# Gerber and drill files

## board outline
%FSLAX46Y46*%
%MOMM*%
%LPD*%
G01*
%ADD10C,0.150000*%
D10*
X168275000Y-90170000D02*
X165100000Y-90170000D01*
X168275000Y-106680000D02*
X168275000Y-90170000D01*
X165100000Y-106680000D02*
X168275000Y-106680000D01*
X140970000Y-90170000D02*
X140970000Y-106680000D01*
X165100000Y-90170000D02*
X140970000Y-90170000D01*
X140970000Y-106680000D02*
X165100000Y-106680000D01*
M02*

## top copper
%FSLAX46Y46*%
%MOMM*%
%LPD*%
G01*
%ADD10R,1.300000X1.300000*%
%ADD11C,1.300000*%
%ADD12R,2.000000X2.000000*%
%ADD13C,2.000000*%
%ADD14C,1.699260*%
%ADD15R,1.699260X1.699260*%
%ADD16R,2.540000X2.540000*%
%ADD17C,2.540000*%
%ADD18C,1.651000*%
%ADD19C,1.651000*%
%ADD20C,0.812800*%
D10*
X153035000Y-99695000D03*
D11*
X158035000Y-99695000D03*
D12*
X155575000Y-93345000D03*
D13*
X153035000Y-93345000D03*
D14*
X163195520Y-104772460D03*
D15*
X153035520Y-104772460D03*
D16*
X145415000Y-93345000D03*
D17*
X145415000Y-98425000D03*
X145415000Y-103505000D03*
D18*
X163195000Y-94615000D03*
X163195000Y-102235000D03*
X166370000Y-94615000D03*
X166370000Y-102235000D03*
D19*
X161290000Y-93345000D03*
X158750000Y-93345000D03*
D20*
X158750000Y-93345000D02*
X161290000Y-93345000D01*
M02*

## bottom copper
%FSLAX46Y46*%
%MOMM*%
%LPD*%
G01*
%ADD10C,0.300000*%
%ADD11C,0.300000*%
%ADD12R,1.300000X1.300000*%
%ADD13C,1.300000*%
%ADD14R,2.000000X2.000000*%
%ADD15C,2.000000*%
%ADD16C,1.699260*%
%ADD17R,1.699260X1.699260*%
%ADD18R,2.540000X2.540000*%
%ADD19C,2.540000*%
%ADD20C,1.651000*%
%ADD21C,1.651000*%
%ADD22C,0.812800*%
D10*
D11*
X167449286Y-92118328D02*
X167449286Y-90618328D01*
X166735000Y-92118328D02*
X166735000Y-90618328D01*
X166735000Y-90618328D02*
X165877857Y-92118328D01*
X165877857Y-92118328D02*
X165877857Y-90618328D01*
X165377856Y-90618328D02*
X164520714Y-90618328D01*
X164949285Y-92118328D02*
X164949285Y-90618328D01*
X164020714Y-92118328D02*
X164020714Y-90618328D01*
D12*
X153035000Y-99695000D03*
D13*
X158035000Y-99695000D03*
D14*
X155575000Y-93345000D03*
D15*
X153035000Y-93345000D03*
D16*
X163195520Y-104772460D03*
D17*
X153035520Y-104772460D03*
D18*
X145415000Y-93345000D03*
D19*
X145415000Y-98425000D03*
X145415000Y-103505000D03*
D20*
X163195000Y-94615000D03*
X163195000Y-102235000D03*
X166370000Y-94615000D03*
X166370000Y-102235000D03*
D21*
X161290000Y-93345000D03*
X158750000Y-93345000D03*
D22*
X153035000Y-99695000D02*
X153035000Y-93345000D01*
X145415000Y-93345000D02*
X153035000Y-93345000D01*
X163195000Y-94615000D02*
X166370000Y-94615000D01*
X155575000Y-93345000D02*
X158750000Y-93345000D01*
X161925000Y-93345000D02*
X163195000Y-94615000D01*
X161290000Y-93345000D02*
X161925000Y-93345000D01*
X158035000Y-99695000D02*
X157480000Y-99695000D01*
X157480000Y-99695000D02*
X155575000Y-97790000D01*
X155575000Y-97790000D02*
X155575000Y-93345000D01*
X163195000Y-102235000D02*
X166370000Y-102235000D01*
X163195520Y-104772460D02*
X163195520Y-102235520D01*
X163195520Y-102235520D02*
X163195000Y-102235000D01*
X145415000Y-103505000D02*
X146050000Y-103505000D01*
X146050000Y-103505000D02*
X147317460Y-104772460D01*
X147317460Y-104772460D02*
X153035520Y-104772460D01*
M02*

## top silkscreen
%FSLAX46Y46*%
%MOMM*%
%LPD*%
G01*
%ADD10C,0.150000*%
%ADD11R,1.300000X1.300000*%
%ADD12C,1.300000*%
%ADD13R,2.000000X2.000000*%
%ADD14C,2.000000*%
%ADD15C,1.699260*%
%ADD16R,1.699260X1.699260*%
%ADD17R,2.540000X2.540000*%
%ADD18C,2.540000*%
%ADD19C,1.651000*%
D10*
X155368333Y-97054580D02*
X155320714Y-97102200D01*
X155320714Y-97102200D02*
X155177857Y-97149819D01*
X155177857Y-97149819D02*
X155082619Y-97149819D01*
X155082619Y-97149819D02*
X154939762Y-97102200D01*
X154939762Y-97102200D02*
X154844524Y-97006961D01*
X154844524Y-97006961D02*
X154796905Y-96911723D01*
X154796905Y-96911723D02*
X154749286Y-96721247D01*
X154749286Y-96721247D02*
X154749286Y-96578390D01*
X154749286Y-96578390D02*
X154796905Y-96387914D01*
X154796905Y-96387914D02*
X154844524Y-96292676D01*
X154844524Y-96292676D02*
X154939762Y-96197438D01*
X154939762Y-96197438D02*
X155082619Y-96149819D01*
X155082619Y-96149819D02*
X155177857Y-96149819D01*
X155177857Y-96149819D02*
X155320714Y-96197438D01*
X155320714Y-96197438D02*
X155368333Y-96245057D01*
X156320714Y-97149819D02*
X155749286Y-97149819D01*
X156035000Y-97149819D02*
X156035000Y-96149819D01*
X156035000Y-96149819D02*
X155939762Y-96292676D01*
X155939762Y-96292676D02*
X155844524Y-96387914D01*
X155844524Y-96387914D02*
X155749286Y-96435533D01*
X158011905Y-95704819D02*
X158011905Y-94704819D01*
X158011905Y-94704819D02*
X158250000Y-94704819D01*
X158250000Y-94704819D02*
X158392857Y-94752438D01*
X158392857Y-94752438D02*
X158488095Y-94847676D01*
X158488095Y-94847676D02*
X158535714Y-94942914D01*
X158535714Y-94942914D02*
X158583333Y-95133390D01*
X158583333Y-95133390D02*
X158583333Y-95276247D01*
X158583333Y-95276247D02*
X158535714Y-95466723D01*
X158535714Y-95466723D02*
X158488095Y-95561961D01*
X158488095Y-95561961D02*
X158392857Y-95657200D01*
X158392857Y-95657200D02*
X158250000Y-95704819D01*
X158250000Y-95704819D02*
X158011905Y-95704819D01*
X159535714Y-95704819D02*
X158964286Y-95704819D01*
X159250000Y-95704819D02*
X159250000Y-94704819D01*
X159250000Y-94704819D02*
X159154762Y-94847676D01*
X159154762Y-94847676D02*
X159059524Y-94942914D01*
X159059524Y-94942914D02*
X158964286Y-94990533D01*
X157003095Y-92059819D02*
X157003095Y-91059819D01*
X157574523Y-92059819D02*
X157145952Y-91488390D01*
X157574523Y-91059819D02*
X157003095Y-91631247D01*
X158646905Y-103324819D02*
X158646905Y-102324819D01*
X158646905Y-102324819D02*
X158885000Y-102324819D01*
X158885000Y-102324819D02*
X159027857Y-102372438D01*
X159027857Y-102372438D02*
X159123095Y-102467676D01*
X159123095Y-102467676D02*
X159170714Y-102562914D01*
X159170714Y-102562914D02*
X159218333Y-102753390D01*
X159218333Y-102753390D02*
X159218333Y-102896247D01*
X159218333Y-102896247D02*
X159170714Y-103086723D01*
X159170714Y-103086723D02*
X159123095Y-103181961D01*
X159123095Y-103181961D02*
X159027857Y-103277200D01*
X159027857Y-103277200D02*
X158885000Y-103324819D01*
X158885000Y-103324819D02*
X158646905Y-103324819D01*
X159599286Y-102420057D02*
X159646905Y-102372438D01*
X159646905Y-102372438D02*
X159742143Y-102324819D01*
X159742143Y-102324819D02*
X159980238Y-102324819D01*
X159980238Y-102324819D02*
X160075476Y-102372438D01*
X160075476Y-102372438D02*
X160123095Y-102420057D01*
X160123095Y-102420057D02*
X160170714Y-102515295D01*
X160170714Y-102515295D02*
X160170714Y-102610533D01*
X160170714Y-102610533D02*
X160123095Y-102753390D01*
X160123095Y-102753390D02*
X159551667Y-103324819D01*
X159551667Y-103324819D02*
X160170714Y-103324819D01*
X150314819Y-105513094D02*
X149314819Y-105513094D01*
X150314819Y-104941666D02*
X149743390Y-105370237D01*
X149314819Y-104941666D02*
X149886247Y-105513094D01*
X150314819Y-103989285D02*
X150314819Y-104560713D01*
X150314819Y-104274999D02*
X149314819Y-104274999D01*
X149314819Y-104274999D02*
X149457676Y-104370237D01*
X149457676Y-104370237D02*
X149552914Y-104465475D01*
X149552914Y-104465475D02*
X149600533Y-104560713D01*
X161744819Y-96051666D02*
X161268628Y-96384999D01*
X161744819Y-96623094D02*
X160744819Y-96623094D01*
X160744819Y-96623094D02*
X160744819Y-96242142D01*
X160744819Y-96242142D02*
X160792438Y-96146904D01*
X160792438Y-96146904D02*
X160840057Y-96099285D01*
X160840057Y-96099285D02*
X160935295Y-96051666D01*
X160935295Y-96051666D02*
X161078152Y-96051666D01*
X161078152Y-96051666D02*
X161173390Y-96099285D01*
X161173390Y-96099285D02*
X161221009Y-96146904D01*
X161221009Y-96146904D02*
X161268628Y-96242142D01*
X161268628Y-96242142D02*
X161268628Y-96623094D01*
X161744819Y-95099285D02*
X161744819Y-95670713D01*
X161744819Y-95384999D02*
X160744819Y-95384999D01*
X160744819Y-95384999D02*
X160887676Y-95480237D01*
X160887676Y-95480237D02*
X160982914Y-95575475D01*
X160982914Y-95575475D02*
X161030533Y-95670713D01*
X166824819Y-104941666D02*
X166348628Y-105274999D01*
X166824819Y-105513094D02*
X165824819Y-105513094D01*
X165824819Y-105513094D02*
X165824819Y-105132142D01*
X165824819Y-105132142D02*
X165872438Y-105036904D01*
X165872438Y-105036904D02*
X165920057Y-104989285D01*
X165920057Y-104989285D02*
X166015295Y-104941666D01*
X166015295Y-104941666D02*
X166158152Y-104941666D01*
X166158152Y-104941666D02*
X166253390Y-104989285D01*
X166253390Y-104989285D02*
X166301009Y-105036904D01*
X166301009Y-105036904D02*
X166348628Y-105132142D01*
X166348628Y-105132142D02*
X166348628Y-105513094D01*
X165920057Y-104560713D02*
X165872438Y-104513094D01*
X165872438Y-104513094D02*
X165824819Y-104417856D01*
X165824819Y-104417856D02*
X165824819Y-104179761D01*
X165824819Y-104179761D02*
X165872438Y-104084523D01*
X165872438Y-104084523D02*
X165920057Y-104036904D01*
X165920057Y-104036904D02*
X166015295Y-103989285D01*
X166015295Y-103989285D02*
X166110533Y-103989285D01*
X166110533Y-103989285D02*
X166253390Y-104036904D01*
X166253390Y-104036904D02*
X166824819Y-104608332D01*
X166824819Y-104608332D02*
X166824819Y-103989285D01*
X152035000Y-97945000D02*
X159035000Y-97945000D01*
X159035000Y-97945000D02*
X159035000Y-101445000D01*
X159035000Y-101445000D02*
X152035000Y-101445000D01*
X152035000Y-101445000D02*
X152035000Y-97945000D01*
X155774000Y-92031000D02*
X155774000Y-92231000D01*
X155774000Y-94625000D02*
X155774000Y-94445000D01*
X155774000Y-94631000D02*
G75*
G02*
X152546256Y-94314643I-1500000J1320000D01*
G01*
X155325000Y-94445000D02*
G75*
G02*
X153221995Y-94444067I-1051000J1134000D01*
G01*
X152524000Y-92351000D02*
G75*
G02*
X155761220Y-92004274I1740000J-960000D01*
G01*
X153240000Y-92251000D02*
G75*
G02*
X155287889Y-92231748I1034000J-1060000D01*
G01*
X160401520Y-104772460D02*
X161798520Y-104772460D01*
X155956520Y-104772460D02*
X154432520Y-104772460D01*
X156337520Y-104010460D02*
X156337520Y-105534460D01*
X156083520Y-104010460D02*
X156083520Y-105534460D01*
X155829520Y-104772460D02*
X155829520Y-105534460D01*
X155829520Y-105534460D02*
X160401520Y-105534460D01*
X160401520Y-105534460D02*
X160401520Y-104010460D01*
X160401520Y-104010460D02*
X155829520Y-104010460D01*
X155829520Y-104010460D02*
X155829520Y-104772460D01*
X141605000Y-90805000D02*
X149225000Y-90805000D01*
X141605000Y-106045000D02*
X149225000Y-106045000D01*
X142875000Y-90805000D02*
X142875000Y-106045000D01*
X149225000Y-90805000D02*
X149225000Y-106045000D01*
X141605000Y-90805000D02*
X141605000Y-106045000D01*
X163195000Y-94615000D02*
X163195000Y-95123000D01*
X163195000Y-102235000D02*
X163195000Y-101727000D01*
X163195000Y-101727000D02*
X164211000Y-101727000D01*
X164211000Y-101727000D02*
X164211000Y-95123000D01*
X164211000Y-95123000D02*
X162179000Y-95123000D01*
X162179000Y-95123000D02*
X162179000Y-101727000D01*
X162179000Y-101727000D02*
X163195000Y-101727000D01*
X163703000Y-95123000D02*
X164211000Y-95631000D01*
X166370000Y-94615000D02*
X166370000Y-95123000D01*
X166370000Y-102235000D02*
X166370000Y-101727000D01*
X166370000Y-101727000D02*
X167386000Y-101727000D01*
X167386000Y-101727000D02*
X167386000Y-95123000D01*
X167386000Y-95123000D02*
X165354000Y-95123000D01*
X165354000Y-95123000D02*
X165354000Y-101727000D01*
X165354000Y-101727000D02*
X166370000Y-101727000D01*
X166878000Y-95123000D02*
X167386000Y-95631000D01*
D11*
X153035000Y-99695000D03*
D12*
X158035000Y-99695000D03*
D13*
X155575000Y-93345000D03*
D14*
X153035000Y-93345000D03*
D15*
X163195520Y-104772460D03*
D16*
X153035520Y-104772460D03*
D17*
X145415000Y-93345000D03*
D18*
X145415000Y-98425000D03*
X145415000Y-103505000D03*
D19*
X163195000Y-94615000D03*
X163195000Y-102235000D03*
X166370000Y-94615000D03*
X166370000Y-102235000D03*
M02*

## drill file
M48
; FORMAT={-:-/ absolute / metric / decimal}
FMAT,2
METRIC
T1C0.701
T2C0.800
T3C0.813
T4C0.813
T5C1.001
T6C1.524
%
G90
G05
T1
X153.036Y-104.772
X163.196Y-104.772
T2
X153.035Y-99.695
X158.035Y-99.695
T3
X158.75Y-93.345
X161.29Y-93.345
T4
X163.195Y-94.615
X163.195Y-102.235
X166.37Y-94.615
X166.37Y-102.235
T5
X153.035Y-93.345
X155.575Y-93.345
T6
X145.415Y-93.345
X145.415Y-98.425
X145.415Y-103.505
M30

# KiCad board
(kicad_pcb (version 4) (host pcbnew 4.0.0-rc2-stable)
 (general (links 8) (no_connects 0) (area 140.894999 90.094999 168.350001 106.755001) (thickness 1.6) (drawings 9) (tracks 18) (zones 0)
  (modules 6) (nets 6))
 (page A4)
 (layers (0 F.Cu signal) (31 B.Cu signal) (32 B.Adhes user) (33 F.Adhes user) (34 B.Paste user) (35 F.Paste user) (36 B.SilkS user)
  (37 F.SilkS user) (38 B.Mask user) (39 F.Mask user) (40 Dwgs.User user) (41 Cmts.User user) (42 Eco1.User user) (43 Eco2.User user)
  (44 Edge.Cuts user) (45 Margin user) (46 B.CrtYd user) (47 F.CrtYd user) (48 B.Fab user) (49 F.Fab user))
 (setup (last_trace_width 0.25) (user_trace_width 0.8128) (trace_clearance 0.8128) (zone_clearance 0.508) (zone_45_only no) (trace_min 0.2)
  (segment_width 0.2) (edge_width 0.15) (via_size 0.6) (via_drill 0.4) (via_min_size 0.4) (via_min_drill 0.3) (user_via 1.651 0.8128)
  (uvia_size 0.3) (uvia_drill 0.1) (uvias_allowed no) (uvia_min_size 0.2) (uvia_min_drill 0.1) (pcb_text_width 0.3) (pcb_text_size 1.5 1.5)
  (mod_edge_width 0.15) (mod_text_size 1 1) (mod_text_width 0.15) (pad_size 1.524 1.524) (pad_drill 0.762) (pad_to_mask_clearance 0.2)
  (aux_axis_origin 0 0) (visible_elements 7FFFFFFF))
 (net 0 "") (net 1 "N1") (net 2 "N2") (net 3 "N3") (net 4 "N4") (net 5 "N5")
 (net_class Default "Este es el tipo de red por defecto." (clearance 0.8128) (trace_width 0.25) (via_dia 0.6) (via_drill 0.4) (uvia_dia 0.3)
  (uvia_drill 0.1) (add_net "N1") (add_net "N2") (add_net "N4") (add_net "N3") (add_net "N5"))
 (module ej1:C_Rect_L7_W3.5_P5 (layer F.Cu) (at 153.035 99.695)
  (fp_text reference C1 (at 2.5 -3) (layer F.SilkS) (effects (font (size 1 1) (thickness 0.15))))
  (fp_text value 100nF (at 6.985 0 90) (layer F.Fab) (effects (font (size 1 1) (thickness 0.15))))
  (fp_line (start -1 -1.75) (end 6 -1.75) (layer F.SilkS) (width 0.15))
  (fp_line (start 6 -1.75) (end 6 1.75) (layer F.SilkS) (width 0.15))
  (fp_line (start 6 1.75) (end -1 1.75) (layer F.SilkS) (width 0.15))
  (fp_line (start -1 1.75) (end -1 -1.75) (layer F.SilkS) (width 0.15))
  (pad 1 thru_hole rect (at 0 0) (size 1.3 1.3) (drill 0.8) (layers *.Cu *.Mask F.SilkS) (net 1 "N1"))
  (pad 2 thru_hole circle (at 5 0) (size 1.3 1.3) (drill 0.8) (layers *.Cu *.Mask F.SilkS) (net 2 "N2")))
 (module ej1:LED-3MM (layer F.Cu) (at 155.575 93.345 180)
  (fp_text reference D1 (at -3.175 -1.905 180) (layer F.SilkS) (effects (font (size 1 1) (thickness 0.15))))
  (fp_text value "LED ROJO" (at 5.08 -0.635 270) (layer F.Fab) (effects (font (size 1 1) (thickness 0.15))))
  (fp_line (start -0.199 1.314) (end -0.199 1.114) (layer F.SilkS) (width 0.15))
  (fp_line (start -0.199 -1.28) (end -0.199 -1.1) (layer F.SilkS) (width 0.15))
  (fp_arc (start 1.301 0.034) (end -0.199 -1.286) (angle 108.5) (layer F.SilkS) (width 0.15))
  (fp_arc (start 1.301 0.034) (end 0.25 -1.1) (angle 85.7) (layer F.SilkS) (width 0.15))
  (fp_arc (start 1.311 0.034) (end 3.051 0.994) (angle 110) (layer F.SilkS) (width 0.15))
  (fp_arc (start 1.301 0.034) (end 2.335 1.094) (angle 87.5) (layer F.SilkS) (width 0.15))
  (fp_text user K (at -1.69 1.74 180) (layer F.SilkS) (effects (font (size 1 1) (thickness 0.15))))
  (pad 1 thru_hole rect (at 0 0 270) (size 2 2) (drill 1.00076) (layers *.Cu *.Mask F.SilkS) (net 2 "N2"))
  (pad 2 thru_hole circle (at 2.54 0 180) (size 2 2) (drill 1.00076) (layers *.Cu *.Mask F.SilkS) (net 1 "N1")))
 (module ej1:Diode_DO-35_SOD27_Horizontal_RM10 (layer F.Cu) (at 153.035 104.775)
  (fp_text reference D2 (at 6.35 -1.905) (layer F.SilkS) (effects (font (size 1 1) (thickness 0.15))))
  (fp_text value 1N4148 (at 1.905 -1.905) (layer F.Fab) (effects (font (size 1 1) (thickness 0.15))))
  (fp_line (start 7.36652 -0.00254) (end 8.76352 -0.00254) (layer F.SilkS) (width 0.15))
  (fp_line (start 2.92152 -0.00254) (end 1.39752 -0.00254) (layer F.SilkS) (width 0.15))
  (fp_line (start 3.30252 -0.76454) (end 3.30252 0.75946) (layer F.SilkS) (width 0.15))
  (fp_line (start 3.04852 -0.76454) (end 3.04852 0.75946) (layer F.SilkS) (width 0.15))
  (fp_line (start 2.79452 -0.00254) (end 2.79452 0.75946) (layer F.SilkS) (width 0.15))
  (fp_line (start 2.79452 0.75946) (end 7.36652 0.75946) (layer F.SilkS) (width 0.15))
  (fp_line (start 7.36652 0.75946) (end 7.36652 -0.76454) (layer F.SilkS) (width 0.15))
  (fp_line (start 7.36652 -0.76454) (end 2.79452 -0.76454) (layer F.SilkS) (width 0.15))
  (fp_line (start 2.79452 -0.76454) (end 2.79452 -0.00254) (layer F.SilkS) (width 0.15))
  (pad 2 thru_hole circle (at 10.16052 -0.00254 180) (size 1.69926 1.69926) (drill 0.70104) (layers *.Cu *.Mask F.SilkS) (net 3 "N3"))
  (pad 1 thru_hole rect (at 0.00052 -0.00254 180) (size 1.69926 1.69926) (drill 0.70104) (layers *.Cu *.Mask F.SilkS) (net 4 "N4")))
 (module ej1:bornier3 (layer F.Cu) (at 145.415 98.425 270)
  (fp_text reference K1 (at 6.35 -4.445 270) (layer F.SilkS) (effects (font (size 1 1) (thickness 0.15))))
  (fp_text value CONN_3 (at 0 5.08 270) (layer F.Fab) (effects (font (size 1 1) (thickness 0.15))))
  (fp_line (start -7.62 3.81) (end -7.62 -3.81) (layer F.SilkS) (width 0.15))
  (fp_line (start 7.62 3.81) (end 7.62 -3.81) (layer F.SilkS) (width 0.15))
  (fp_line (start -7.62 2.54) (end 7.62 2.54) (layer F.SilkS) (width 0.15))
  (fp_line (start -7.62 -3.81) (end 7.62 -3.81) (layer F.SilkS) (width 0.15))
  (fp_line (start -7.62 3.81) (end 7.62 3.81) (layer F.SilkS) (width 0.15))
  (pad 1 thru_hole rect (at -5.08 0 270) (size 2.54 2.54) (drill 1.524) (layers *.Cu *.Mask F.SilkS) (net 1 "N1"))
  (pad 2 thru_hole circle (at 0 0 270) (size 2.54 2.54) (drill 1.524) (layers *.Cu *.Mask F.SilkS) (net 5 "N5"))
  (pad 3 thru_hole circle (at 5.08 0 270) (size 2.54 2.54) (drill 1.524) (layers *.Cu *.Mask F.SilkS) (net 4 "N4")))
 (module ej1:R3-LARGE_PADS (layer F.Cu) (at 163.195 98.425 270)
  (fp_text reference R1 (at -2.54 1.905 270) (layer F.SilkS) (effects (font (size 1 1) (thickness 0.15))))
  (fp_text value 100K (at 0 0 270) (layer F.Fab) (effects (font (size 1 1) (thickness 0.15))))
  (fp_line (start -3.81 0) (end -3.302 0) (layer F.SilkS) (width 0.15))
  (fp_line (start 3.81 0) (end 3.302 0) (layer F.SilkS) (width 0.15))
  (fp_line (start 3.302 0) (end 3.302 -1.016) (layer F.SilkS) (width 0.15))
  (fp_line (start 3.302 -1.016) (end -3.302 -1.016) (layer F.SilkS) (width 0.15))
  (fp_line (start -3.302 -1.016) (end -3.302 1.016) (layer F.SilkS) (width 0.15))
  (fp_line (start -3.302 1.016) (end 3.302 1.016) (layer F.SilkS) (width 0.15))
  (fp_line (start 3.302 1.016) (end 3.302 0) (layer F.SilkS) (width 0.15))
  (fp_line (start -3.302 -0.508) (end -2.794 -1.016) (layer F.SilkS) (width 0.15))
  (pad 1 thru_hole circle (at -3.81 0 270) (size 1.651 1.651) (drill 0.8128) (layers *.Cu *.Mask F.SilkS) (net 2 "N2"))
  (pad 2 thru_hole circle (at 3.81 0 270) (size 1.651 1.651) (drill 0.8128) (layers *.Cu *.Mask F.SilkS) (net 3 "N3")))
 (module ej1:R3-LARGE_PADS (layer F.Cu) (at 166.37 98.425 270)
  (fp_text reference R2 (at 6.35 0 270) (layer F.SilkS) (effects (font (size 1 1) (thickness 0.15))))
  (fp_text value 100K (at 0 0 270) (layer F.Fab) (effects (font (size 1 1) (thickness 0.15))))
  (fp_line (start -3.81 0) (end -3.302 0) (layer F.SilkS) (width 0.15))
  (fp_line (start 3.81 0) (end 3.302 0) (layer F.SilkS) (width 0.15))
  (fp_line (start 3.302 0) (end 3.302 -1.016) (layer F.SilkS) (width 0.15))
  (fp_line (start 3.302 -1.016) (end -3.302 -1.016) (layer F.SilkS) (width 0.15))
  (fp_line (start -3.302 -1.016) (end -3.302 1.016) (layer F.SilkS) (width 0.15))
  (fp_line (start -3.302 1.016) (end 3.302 1.016) (layer F.SilkS) (width 0.15))
  (fp_line (start 3.302 1.016) (end 3.302 0) (layer F.SilkS) (width 0.15))
  (fp_line (start -3.302 -0.508) (end -2.794 -1.016) (layer F.SilkS) (width 0.15))
  (pad 1 thru_hole circle (at -3.81 0 270) (size 1.651 1.651) (drill 0.8128) (layers *.Cu *.Mask F.SilkS) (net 2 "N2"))
  (pad 2 thru_hole circle (at 3.81 0 270) (size 1.651 1.651) (drill 0.8128) (layers *.Cu *.Mask F.SilkS) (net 3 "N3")))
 (gr_line (start 168.275 90.17) (end 165.1 90.17) (angle 90) (layer Edge.Cuts) (width 0.15))
 (gr_line (start 168.275 106.68) (end 168.275 90.17) (angle 90) (layer Edge.Cuts) (width 0.15))
 (gr_line (start 165.1 106.68) (end 168.275 106.68) (angle 90) (layer Edge.Cuts) (width 0.15))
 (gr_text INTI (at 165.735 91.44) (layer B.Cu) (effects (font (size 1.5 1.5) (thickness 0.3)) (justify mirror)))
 (gr_line (start 140.97 90.17) (end 140.97 106.68) (angle 90) (layer Edge.Cuts) (width 0.15))
 (gr_line (start 165.1 90.17) (end 140.97 90.17) (angle 90) (layer Edge.Cuts) (width 0.15))
 (gr_line (start 140.97 106.68) (end 165.1 106.68) (angle 90) (layer Edge.Cuts) (width 0.15))
 (segment (start 153.035 99.695) (end 153.035 93.345) (width 0.8128) (layer B.Cu) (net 1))
 (segment (start 145.415 93.345) (end 153.035 93.345) (width 0.8128) (layer B.Cu) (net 1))
 (segment (start 163.195 94.615) (end 166.37 94.615) (width 0.8128) (layer B.Cu) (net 2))
 (segment (start 155.575 93.345) (end 158.75 93.345) (width 0.8128) (layer B.Cu) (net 2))
 (segment (start 161.925 93.345) (end 163.195 94.615) (width 0.8128) (layer B.Cu) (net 2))
 (segment (start 161.29 93.345) (end 161.925 93.345) (width 0.8128) (layer B.Cu) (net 2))
 (via (at 161.29 93.345) (size 1.651) (drill 0.8128) (layers F.Cu B.Cu) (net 2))
 (segment (start 158.75 93.345) (end 161.29 93.345) (width 0.8128) (layer F.Cu) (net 2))
 (via (at 158.75 93.345) (size 1.651) (drill 0.8128) (layers F.Cu B.Cu) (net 2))
 (segment (start 158.035 99.695) (end 157.48 99.695) (width 0.8128) (layer B.Cu) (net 2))
 (segment (start 157.48 99.695) (end 155.575 97.79) (width 0.8128) (layer B.Cu) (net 2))
 (segment (start 155.575 97.79) (end 155.575 93.345) (width 0.8128) (layer B.Cu) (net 2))
 (segment (start 163.195 102.235) (end 166.37 102.235) (width 0.8128) (layer B.Cu) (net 3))
 (segment (start 163.19552 104.77246) (end 163.19552 102.23552) (width 0.8128) (layer B.Cu) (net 3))
 (segment (start 163.19552 102.23552) (end 163.195 102.235) (width 0.8128) (layer B.Cu) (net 3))
 (segment (start 145.415 103.505) (end 146.05 103.505) (width 0.8128) (layer B.Cu) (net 4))
 (segment (start 146.05 103.505) (end 147.31746 104.77246) (width 0.8128) (layer B.Cu) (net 4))
 (segment (start 147.31746 104.77246) (end 153.03552 104.77246) (width 0.8128) (layer B.Cu) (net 4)))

